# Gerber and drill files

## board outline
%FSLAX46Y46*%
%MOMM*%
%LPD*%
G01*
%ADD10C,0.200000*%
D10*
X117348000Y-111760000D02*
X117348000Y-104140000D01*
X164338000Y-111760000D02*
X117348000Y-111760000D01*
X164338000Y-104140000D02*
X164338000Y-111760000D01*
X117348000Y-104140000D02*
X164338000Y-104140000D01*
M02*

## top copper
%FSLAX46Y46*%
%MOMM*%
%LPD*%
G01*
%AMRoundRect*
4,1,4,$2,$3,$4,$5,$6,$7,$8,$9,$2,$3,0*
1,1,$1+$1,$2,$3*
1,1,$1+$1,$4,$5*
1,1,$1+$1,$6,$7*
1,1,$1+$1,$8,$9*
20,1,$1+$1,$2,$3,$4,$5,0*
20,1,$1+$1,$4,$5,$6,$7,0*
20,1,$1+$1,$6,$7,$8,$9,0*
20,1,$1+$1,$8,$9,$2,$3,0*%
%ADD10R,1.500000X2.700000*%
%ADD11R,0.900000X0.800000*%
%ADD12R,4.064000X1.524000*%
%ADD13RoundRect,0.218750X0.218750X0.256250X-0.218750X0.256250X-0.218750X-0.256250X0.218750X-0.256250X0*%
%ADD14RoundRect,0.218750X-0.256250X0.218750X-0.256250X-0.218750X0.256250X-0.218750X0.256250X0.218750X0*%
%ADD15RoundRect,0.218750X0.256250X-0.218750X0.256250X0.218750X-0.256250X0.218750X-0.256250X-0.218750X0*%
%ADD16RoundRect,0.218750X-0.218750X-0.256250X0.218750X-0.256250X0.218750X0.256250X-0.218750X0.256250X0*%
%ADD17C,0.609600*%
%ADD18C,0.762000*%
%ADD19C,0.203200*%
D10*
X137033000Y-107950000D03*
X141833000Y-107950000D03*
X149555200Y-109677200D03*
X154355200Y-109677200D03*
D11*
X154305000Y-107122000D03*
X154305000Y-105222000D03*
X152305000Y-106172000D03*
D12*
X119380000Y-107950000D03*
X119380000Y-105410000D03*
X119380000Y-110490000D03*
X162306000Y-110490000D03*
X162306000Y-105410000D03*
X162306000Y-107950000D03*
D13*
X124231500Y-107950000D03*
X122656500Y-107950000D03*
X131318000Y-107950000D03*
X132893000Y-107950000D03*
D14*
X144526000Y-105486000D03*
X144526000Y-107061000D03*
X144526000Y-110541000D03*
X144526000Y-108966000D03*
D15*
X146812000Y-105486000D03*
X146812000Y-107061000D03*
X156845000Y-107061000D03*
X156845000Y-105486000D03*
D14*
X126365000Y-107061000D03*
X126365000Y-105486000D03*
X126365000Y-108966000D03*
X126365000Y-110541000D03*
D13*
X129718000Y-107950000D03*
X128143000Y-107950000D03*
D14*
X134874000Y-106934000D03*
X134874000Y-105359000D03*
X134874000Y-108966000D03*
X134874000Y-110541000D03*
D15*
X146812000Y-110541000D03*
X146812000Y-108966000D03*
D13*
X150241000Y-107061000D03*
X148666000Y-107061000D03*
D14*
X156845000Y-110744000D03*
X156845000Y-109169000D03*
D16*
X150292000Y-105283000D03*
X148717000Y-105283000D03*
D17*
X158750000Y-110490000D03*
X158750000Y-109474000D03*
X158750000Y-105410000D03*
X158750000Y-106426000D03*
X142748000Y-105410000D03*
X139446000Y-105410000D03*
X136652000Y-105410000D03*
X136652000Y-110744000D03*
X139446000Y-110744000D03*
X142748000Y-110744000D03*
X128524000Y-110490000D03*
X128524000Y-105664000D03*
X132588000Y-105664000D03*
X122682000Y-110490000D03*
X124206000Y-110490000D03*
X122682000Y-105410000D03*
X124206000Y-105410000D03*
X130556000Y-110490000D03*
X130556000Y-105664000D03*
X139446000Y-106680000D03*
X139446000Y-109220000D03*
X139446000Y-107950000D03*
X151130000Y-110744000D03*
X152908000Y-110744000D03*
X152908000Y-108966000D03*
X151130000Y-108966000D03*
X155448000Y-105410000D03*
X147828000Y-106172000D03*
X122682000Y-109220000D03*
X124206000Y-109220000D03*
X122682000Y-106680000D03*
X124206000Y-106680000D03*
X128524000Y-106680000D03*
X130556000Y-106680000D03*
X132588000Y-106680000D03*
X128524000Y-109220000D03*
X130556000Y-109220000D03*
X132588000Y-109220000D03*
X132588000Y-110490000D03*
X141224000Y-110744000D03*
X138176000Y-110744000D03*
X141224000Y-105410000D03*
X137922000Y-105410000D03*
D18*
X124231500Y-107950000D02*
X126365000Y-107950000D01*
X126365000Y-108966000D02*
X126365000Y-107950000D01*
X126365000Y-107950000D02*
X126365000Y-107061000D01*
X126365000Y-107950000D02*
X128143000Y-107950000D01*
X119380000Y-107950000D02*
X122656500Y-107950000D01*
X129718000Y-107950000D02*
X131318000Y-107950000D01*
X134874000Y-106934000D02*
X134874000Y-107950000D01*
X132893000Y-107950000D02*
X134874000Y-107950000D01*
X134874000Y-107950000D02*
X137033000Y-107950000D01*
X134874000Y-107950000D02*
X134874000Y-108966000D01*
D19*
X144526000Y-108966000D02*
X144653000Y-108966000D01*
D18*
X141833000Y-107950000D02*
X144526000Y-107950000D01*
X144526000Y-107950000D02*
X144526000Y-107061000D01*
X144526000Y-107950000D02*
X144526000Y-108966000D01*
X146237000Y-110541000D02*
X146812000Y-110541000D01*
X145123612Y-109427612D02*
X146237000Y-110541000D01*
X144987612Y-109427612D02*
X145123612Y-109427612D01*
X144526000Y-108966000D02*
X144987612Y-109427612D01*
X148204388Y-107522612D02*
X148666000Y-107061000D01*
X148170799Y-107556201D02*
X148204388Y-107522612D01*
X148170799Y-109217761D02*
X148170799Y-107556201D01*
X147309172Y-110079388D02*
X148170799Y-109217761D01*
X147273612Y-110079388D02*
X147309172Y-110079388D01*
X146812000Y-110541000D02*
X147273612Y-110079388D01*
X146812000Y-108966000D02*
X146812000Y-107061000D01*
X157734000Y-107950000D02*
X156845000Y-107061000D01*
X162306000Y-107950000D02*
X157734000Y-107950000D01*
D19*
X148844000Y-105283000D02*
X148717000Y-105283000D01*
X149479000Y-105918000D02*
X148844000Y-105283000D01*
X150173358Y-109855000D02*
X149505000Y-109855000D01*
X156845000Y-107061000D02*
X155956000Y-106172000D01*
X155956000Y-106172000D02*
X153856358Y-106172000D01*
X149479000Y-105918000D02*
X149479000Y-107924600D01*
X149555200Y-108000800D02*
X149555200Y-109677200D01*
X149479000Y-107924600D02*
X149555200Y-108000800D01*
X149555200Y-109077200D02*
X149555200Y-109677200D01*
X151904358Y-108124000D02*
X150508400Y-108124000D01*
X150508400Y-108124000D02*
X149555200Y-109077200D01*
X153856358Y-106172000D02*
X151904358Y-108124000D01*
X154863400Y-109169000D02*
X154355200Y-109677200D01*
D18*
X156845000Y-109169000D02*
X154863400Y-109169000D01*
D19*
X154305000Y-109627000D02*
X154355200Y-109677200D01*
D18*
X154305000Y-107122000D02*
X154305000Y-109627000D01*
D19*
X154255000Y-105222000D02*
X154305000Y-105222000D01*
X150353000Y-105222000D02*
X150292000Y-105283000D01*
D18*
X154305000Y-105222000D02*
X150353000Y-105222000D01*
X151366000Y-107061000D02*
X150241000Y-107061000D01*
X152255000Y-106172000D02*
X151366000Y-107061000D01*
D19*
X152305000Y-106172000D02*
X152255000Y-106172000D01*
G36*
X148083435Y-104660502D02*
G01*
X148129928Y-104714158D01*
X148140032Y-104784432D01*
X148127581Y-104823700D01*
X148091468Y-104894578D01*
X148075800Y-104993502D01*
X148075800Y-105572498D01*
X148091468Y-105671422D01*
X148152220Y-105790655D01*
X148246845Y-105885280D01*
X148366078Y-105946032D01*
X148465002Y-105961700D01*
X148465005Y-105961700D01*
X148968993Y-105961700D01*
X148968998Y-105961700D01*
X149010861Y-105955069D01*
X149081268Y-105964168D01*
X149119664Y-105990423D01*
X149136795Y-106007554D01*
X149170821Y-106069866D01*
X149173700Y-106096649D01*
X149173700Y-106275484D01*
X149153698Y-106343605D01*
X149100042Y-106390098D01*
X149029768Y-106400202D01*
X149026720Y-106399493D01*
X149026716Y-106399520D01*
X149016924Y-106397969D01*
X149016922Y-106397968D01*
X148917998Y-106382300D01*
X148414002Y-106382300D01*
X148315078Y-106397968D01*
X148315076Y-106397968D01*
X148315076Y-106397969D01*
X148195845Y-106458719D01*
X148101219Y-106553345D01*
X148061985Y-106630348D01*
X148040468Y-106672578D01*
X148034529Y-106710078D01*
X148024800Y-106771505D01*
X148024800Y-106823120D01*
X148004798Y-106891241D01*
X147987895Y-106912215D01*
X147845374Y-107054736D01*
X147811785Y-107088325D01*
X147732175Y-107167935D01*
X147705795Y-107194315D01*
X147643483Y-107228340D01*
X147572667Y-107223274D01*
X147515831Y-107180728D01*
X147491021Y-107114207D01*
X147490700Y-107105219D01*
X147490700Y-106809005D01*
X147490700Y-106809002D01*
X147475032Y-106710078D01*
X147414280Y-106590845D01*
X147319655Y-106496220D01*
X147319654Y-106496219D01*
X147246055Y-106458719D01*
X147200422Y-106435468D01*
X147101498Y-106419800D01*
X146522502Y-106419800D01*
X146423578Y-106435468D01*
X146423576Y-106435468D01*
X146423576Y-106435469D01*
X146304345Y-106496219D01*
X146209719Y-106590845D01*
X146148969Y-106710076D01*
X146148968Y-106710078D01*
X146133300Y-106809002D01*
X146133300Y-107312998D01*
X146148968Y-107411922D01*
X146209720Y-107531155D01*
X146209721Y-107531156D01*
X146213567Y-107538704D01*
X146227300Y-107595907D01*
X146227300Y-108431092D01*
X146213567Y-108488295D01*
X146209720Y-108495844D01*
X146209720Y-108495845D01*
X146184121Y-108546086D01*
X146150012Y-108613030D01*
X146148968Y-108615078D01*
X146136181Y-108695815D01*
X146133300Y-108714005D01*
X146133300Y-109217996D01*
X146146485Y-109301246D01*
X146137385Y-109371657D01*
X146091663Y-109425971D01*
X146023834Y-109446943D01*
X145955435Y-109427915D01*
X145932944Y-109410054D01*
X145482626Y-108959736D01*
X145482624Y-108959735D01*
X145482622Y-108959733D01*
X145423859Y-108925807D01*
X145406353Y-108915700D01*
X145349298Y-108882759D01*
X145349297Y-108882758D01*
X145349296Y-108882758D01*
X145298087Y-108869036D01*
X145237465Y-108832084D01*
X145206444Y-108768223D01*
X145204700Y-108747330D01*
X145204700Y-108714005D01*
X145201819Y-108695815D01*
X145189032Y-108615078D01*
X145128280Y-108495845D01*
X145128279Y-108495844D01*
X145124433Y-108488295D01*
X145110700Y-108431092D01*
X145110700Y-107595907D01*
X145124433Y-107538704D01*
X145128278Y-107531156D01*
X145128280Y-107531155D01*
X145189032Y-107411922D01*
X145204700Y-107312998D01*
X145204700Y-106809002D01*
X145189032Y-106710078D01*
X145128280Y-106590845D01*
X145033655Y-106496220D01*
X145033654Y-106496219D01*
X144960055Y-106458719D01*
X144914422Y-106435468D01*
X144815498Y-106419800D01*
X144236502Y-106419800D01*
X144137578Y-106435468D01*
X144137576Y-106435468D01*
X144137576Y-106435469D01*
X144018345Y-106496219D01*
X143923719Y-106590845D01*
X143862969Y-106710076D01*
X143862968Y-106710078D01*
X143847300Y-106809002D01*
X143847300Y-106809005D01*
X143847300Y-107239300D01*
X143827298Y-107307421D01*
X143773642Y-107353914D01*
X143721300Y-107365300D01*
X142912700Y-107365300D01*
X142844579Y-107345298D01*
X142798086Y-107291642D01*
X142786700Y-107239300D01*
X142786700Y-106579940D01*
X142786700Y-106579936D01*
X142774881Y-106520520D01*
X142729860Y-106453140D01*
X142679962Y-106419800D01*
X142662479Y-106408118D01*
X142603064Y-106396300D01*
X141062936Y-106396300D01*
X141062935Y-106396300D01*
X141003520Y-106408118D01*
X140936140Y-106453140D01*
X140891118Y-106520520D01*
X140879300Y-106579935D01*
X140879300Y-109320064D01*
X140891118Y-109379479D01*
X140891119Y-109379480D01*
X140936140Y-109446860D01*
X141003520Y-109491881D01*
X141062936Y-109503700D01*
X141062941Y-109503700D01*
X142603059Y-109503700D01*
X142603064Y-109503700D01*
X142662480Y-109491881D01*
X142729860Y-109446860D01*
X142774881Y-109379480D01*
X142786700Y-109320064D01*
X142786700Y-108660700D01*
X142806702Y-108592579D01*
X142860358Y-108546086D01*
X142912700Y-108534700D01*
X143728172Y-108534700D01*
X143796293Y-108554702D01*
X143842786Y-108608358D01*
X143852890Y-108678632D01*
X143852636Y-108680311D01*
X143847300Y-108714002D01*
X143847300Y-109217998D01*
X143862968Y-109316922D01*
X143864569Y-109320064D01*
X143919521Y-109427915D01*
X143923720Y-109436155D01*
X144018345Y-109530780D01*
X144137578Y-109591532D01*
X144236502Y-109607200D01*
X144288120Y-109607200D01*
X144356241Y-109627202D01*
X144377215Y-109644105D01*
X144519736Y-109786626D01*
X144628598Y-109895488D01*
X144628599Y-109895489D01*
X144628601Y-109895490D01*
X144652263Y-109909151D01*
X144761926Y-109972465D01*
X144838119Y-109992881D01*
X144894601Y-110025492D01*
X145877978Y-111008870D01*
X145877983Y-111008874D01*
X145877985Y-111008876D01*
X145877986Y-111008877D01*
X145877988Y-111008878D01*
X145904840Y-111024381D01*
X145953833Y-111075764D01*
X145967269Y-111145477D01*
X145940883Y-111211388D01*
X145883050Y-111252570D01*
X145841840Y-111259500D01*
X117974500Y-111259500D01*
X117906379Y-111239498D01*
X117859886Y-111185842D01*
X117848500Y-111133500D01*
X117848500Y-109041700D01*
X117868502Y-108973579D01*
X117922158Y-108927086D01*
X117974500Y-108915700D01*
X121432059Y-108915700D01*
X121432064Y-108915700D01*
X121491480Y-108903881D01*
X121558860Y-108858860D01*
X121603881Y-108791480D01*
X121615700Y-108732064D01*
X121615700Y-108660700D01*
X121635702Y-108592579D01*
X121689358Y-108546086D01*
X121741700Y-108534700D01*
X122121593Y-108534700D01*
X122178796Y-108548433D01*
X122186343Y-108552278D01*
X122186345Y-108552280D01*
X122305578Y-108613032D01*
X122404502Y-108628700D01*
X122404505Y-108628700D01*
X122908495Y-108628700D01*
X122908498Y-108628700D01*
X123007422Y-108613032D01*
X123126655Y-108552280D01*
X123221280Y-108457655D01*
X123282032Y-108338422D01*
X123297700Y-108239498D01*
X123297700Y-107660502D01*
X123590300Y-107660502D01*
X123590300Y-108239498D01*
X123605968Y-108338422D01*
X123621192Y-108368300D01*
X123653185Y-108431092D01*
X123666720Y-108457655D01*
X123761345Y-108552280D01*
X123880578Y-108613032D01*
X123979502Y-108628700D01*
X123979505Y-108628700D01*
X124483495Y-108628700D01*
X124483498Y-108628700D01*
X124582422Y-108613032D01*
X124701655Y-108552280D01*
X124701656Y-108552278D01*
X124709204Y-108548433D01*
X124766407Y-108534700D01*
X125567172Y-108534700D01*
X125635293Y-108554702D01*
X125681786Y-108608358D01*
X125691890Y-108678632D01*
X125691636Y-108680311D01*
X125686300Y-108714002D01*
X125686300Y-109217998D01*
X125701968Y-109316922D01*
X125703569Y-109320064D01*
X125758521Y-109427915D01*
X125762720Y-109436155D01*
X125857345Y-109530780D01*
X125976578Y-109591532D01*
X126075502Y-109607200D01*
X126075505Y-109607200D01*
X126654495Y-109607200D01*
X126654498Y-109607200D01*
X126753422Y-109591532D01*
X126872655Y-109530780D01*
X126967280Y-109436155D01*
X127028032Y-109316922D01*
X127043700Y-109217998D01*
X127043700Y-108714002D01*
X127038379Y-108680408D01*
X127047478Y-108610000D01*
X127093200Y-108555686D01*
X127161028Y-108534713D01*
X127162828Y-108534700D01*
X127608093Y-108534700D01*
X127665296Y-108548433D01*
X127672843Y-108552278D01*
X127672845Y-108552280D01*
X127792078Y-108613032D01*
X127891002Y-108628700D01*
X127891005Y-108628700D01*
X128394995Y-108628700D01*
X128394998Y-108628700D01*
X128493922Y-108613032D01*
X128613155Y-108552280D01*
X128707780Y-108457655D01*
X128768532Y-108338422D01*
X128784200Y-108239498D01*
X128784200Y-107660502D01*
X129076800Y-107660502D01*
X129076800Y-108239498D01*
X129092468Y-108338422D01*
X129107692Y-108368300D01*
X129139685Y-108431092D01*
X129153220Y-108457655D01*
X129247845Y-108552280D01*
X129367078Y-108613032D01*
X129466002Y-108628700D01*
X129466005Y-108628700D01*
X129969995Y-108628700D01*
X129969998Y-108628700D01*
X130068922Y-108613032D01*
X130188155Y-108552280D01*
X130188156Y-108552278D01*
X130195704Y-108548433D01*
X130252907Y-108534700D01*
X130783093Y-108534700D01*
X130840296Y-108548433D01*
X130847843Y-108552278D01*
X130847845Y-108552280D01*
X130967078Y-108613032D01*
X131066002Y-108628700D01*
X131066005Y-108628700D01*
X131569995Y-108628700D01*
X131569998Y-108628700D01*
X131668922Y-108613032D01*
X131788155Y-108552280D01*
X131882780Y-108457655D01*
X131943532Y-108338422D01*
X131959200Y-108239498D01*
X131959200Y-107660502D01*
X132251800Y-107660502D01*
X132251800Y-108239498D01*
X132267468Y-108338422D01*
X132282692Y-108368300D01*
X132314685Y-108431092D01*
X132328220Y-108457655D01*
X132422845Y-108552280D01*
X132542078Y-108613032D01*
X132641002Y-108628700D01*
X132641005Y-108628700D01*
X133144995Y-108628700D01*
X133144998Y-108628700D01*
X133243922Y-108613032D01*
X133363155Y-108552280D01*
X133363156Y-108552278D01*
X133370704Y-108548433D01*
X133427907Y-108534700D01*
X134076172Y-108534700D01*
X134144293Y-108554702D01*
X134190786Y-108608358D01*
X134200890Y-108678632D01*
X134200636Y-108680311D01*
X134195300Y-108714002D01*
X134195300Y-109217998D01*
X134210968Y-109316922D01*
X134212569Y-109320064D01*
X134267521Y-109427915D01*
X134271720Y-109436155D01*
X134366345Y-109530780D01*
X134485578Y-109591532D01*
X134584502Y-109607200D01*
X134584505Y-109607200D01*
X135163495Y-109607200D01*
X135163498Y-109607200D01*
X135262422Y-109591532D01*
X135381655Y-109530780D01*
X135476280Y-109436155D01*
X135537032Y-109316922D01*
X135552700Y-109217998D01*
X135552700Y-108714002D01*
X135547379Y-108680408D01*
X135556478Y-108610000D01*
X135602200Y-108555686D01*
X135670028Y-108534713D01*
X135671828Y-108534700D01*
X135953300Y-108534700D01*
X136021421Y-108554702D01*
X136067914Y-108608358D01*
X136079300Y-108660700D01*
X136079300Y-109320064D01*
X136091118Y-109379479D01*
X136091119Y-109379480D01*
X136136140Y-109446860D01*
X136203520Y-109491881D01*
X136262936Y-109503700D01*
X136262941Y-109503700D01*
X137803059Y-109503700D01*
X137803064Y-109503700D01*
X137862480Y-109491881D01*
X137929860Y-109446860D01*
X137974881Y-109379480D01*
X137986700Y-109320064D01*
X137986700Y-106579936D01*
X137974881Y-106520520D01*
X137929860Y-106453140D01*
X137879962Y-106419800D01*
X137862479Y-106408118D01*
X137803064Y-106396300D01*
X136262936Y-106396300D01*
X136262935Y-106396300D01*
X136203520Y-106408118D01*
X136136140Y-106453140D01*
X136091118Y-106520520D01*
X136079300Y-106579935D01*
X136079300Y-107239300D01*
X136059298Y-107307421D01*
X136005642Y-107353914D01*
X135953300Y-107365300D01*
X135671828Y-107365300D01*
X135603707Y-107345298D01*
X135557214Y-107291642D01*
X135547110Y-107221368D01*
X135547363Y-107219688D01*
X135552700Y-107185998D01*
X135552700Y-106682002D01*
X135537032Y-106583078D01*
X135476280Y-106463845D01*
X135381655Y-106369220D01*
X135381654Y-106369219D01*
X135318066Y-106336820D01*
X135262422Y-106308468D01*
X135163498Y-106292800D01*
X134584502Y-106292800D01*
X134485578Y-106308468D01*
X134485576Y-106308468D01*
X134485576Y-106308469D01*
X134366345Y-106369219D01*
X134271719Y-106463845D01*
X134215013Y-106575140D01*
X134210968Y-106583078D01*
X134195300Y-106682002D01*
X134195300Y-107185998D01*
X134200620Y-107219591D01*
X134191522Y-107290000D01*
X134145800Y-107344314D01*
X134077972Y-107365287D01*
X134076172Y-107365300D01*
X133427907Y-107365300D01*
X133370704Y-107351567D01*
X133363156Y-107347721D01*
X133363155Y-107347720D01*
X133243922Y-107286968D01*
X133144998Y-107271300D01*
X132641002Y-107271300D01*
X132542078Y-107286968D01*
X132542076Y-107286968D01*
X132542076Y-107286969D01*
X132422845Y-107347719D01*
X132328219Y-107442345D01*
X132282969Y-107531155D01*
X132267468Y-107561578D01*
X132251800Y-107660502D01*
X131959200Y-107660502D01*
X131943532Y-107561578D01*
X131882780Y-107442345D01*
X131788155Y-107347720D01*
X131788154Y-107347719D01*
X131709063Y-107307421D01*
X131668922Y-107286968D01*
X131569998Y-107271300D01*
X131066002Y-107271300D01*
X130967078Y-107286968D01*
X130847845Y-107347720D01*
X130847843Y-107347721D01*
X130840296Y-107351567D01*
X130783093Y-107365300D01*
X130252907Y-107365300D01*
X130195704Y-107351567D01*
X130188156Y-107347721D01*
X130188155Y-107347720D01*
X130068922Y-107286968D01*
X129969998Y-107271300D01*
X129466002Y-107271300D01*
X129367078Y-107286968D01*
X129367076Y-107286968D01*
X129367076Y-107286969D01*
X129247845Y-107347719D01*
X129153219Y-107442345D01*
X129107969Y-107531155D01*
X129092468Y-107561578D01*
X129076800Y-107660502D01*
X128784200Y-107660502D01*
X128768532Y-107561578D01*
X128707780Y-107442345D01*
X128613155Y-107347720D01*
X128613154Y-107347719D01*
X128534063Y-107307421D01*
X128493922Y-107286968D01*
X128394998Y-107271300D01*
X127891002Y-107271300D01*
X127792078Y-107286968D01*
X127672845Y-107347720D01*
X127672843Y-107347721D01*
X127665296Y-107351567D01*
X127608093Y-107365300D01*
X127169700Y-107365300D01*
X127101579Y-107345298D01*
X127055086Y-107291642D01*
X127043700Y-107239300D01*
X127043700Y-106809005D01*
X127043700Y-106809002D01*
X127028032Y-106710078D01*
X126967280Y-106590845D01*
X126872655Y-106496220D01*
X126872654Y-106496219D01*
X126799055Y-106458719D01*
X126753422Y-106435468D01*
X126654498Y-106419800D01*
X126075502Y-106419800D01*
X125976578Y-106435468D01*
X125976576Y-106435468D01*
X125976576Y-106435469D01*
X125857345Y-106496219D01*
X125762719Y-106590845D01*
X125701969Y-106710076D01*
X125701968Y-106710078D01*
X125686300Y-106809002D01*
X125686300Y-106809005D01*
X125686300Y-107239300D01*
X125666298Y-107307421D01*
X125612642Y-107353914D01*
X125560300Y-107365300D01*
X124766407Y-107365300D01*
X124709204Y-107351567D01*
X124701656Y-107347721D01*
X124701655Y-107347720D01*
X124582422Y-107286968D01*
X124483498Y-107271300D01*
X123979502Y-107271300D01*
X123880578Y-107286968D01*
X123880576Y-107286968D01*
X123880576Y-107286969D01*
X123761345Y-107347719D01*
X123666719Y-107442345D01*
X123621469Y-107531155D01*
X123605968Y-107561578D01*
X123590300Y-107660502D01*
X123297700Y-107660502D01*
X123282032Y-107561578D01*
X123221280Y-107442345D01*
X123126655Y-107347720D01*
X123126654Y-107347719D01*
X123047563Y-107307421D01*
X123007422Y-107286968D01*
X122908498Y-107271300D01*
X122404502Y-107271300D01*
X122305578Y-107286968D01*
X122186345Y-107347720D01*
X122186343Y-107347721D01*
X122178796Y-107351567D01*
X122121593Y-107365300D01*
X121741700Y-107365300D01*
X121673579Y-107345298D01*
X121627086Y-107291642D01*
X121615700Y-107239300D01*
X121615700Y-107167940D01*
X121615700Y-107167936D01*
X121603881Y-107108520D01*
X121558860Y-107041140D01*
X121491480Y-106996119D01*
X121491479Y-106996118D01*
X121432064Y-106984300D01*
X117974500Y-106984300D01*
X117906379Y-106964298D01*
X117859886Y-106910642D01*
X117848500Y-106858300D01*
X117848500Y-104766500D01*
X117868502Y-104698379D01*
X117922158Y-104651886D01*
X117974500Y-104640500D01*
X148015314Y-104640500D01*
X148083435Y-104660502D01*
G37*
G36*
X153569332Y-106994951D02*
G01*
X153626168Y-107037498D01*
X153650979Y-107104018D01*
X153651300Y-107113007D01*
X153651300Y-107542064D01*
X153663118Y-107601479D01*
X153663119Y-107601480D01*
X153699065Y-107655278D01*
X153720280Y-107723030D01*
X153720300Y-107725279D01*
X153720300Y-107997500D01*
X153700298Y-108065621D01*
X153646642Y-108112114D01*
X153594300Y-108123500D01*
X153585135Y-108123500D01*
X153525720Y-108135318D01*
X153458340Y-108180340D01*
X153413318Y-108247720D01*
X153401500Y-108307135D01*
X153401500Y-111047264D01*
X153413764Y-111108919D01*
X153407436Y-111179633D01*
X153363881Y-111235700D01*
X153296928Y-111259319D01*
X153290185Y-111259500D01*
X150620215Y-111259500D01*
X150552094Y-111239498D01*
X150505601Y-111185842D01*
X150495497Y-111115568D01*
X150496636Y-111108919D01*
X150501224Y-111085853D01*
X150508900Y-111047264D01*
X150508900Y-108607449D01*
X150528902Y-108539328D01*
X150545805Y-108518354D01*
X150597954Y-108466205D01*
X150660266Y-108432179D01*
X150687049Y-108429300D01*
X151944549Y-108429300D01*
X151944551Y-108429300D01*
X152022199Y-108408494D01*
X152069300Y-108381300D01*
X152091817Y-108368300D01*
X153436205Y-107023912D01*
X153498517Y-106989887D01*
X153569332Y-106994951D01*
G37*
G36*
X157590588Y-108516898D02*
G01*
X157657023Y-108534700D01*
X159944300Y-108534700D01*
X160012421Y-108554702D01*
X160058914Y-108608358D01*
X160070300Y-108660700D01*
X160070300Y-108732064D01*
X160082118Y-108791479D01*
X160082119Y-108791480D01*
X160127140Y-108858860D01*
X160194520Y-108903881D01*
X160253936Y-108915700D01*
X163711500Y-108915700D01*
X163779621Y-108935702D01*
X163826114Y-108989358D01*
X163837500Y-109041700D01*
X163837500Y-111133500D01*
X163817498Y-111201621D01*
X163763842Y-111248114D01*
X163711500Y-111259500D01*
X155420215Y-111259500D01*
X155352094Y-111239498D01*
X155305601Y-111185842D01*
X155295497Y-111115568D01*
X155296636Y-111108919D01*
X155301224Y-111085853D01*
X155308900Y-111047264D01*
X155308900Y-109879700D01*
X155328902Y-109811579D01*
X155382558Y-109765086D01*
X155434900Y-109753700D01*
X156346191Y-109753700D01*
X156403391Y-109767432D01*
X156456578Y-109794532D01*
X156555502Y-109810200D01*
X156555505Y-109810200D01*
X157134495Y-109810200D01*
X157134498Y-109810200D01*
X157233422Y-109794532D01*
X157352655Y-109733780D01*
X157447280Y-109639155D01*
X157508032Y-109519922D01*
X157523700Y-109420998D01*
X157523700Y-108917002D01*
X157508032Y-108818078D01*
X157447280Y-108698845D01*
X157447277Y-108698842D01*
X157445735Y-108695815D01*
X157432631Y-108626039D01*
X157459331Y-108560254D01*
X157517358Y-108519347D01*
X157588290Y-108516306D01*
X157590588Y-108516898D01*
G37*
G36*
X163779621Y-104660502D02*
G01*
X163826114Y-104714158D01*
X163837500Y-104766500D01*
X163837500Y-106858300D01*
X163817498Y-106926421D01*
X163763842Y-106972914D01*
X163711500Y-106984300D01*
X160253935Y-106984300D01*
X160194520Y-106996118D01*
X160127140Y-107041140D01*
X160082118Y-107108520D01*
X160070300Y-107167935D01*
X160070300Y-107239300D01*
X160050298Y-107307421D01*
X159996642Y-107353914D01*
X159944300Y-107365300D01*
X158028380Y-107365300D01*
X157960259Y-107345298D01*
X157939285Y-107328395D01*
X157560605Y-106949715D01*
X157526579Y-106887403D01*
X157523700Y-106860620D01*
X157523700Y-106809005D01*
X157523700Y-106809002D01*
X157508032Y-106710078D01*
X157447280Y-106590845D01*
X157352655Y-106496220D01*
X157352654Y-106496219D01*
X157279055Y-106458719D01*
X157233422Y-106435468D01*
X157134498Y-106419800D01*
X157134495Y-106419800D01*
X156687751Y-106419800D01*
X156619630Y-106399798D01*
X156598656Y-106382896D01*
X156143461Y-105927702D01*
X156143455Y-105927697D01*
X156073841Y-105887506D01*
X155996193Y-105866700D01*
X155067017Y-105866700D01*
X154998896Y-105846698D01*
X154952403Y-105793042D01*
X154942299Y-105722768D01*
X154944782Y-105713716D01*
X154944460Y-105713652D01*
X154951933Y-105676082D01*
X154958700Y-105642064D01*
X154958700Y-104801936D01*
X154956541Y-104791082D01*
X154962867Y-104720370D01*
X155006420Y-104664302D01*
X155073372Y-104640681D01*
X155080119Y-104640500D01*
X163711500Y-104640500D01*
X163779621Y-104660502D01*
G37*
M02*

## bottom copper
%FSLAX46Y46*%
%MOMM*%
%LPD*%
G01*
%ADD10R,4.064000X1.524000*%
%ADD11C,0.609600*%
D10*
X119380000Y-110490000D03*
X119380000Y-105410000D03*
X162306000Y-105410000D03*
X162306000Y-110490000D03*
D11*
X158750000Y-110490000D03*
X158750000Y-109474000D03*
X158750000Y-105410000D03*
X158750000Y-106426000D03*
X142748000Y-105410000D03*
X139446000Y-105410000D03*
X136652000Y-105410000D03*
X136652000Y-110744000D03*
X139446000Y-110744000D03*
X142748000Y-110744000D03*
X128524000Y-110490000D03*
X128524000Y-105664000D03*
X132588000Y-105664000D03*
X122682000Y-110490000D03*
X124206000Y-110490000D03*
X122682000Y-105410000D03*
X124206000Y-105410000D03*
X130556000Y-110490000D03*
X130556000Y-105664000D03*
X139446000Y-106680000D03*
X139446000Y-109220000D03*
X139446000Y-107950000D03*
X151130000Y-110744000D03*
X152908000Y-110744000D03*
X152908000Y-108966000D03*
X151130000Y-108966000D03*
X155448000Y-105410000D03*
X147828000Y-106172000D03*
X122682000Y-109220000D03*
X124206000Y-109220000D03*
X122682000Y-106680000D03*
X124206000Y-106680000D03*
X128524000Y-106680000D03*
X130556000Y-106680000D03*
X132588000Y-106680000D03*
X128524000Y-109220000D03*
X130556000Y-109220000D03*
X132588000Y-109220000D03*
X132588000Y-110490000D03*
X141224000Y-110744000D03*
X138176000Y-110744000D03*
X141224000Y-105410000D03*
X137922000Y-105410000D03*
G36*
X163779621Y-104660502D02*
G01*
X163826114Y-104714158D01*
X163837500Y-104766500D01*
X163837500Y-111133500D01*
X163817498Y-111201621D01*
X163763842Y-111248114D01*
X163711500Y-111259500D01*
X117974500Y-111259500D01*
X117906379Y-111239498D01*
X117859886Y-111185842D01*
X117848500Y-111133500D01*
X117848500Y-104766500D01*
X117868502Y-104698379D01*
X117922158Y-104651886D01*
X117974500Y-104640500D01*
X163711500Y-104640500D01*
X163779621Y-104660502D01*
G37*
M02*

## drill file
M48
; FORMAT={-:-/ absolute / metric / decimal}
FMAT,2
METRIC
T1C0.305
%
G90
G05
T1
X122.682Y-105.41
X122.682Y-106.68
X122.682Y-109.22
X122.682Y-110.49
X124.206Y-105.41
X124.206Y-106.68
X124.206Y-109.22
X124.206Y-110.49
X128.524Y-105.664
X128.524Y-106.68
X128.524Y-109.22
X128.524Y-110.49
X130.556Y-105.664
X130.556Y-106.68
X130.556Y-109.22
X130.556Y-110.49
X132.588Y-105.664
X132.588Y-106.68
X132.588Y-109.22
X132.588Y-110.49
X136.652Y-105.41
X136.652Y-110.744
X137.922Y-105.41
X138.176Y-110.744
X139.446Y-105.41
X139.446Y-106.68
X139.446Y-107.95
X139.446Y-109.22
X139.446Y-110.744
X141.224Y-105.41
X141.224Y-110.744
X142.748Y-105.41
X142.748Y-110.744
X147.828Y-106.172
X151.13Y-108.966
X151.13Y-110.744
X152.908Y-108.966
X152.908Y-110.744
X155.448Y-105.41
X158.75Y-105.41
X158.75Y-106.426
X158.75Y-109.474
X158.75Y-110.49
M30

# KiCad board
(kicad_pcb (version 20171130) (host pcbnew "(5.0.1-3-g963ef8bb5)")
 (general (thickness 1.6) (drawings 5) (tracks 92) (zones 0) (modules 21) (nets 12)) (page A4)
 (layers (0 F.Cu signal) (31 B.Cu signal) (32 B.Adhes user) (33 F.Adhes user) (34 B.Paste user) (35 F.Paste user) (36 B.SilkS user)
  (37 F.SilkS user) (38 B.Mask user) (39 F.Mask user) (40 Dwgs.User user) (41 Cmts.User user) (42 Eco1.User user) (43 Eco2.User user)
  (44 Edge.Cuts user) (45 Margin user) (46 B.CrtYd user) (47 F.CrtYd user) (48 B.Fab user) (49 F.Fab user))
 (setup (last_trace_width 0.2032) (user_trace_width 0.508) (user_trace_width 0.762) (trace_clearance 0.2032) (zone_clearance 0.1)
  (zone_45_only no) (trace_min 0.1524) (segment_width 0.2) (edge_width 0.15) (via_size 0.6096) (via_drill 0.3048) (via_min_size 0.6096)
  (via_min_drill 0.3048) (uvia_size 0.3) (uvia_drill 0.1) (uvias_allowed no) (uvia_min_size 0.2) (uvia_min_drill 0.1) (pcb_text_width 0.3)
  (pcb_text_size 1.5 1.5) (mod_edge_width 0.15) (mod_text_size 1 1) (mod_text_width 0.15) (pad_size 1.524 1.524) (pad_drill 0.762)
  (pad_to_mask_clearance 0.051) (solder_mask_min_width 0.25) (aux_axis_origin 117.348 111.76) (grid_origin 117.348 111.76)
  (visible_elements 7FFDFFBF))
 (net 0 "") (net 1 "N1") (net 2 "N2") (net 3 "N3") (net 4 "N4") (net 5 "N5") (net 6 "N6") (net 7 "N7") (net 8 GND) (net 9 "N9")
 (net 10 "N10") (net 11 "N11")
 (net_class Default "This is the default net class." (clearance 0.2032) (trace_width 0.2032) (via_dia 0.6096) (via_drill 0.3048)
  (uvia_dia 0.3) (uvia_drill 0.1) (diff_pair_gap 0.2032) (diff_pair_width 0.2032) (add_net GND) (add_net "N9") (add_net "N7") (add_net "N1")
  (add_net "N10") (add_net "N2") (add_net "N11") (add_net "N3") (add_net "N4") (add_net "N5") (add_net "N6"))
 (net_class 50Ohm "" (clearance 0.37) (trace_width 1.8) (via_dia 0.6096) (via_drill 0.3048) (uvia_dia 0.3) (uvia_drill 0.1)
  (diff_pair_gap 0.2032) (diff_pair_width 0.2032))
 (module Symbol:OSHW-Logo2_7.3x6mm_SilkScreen (layer B.Cu) (at 155.194 107.696 180)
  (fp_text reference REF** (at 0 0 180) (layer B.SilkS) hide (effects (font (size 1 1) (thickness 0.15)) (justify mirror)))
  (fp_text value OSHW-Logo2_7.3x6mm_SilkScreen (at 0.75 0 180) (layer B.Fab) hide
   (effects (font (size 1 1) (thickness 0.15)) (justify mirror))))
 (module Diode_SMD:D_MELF (layer F.Cu) (at 139.433 107.95 180)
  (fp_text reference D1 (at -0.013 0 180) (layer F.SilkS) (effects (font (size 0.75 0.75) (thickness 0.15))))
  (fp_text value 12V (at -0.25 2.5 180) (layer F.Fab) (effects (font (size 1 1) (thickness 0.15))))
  (pad 2 smd rect (at 2.4 0 180) (size 1.5 2.7) (layers F.Cu F.Paste F.Mask) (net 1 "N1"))
  (pad 1 smd rect (at -2.4 0 180) (size 1.5 2.7) (layers F.Cu F.Paste F.Mask) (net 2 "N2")))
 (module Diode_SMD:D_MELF (layer F.Cu) (at 151.9552 109.6772)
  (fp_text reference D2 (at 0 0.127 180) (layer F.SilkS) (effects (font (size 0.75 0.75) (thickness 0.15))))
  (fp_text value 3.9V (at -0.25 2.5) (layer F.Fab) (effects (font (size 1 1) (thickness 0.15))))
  (pad 1 smd rect (at -2.4 0) (size 1.5 2.7) (layers F.Cu F.Paste F.Mask) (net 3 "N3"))
  (pad 2 smd rect (at 2.4 0) (size 1.5 2.7) (layers F.Cu F.Paste F.Mask) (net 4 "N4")))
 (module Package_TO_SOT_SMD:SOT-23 (layer F.Cu) (at 153.305 106.172 180)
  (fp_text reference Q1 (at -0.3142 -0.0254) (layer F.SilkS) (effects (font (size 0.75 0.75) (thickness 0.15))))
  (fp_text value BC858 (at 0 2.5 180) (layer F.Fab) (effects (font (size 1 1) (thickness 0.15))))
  (pad 1 smd rect (at -1 -0.95 180) (size 0.9 0.8) (layers F.Cu F.Paste F.Mask) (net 4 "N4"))
  (pad 2 smd rect (at -1 0.95 180) (size 0.9 0.8) (layers F.Cu F.Paste F.Mask) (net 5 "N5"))
  (pad 3 smd rect (at 1 0 180) (size 0.9 0.8) (layers F.Cu F.Paste F.Mask) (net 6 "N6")))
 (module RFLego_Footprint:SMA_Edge (layer F.Cu) (at 117.348 107.95)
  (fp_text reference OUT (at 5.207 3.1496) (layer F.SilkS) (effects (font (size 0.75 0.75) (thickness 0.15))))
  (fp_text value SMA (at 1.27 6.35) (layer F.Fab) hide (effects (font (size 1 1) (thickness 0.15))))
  (pad 1 smd rect (at 2.032 0) (size 4.064 1.524) (layers F.Cu F.Mask) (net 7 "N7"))
  (pad 2 smd rect (at 2.032 -2.54) (size 4.064 1.524) (layers F.Cu F.Mask) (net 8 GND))
  (pad 2 smd rect (at 2.032 2.54) (size 4.064 1.524) (layers B.Cu B.Mask) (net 8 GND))
  (pad 2 smd rect (at 2.032 -2.54) (size 4.064 1.524) (layers B.Cu B.Mask) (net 8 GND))
  (pad 2 smd rect (at 2.032 2.54) (size 4.064 1.524) (layers F.Cu F.Mask) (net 8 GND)))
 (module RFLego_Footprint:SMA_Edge (layer F.Cu) (at 160.274 107.95)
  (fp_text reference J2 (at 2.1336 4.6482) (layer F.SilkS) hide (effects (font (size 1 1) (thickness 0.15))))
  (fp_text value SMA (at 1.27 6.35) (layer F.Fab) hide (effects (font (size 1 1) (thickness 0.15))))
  (pad 2 smd rect (at 2.032 2.54) (size 4.064 1.524) (layers F.Cu F.Mask) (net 8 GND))
  (pad 2 smd rect (at 2.032 -2.54) (size 4.064 1.524) (layers B.Cu B.Mask) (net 8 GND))
  (pad 2 smd rect (at 2.032 2.54) (size 4.064 1.524) (layers B.Cu B.Mask) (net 8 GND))
  (pad 2 smd rect (at 2.032 -2.54) (size 4.064 1.524) (layers F.Cu F.Mask) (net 8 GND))
  (pad 1 smd rect (at 2.032 0) (size 4.064 1.524) (layers F.Cu F.Mask) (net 3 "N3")))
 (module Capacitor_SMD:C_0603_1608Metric (layer F.Cu) (at 123.444 107.95 180)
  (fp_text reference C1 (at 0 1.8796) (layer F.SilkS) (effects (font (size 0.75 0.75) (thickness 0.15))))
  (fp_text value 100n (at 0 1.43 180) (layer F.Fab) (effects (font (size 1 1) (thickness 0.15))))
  (pad 1 smd roundrect (at -0.7875 0 180) (size 0.875 0.95) (layers F.Cu F.Paste F.Mask) (roundrect_rratio 0.25) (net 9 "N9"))
  (pad 2 smd roundrect (at 0.7875 0 180) (size 0.875 0.95) (layers F.Cu F.Paste F.Mask) (roundrect_rratio 0.25) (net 7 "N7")))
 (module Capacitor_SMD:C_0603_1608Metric (layer F.Cu) (at 132.1055 107.95 180)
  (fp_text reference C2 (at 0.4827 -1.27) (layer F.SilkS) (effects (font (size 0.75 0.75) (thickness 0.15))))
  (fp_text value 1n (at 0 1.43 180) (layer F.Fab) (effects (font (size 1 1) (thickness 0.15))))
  (pad 2 smd roundrect (at 0.7875 0 180) (size 0.875 0.95) (layers F.Cu F.Paste F.Mask) (roundrect_rratio 0.25) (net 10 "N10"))
  (pad 1 smd roundrect (at -0.7875 0 180) (size 0.875 0.95) (layers F.Cu F.Paste F.Mask) (roundrect_rratio 0.25) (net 1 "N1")))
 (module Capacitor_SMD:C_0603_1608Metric (layer F.Cu) (at 144.526 106.2735 270)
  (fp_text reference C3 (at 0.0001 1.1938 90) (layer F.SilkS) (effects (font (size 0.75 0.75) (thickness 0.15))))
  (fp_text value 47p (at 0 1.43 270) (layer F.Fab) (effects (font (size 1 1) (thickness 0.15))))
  (pad 1 smd roundrect (at -0.7875 0 270) (size 0.875 0.95) (layers F.Cu F.Paste F.Mask) (roundrect_rratio 0.25) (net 8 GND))
  (pad 2 smd roundrect (at 0.7875 0 270) (size 0.875 0.95) (layers F.Cu F.Paste F.Mask) (roundrect_rratio 0.25) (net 2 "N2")))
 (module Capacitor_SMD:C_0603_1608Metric (layer F.Cu) (at 144.526 109.7535 270)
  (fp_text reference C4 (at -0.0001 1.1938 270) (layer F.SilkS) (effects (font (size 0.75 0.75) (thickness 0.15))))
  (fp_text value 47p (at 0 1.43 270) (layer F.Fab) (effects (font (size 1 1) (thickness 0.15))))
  (pad 2 smd roundrect (at 0.7875 0 270) (size 0.875 0.95) (layers F.Cu F.Paste F.Mask) (roundrect_rratio 0.25) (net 8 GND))
  (pad 1 smd roundrect (at -0.7875 0 270) (size 0.875 0.95) (layers F.Cu F.Paste F.Mask) (roundrect_rratio 0.25) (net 2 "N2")))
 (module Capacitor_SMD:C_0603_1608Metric (layer F.Cu) (at 146.812 106.2735 90)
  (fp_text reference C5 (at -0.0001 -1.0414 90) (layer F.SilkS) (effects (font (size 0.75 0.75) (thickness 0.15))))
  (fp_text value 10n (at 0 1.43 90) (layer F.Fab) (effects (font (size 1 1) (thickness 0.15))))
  (pad 2 smd roundrect (at 0.7875 0 90) (size 0.875 0.95) (layers F.Cu F.Paste F.Mask) (roundrect_rratio 0.25) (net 8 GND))
  (pad 1 smd roundrect (at -0.7875 0 90) (size 0.875 0.95) (layers F.Cu F.Paste F.Mask) (roundrect_rratio 0.25) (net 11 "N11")))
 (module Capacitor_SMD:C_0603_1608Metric (layer F.Cu) (at 156.845 106.2735 90)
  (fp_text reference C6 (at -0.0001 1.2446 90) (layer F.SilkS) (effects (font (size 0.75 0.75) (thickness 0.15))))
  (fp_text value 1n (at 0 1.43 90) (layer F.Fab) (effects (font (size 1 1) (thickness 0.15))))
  (pad 1 smd roundrect (at -0.7875 0 90) (size 0.875 0.95) (layers F.Cu F.Paste F.Mask) (roundrect_rratio 0.25) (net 3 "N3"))
  (pad 2 smd roundrect (at 0.7875 0 90) (size 0.875 0.95) (layers F.Cu F.Paste F.Mask) (roundrect_rratio 0.25) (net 8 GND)))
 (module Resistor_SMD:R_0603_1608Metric (layer F.Cu) (at 126.365 106.2735 270)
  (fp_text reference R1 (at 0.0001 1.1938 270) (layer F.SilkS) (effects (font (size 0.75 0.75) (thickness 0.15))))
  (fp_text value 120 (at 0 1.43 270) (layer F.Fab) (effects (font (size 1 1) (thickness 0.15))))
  (pad 2 smd roundrect (at 0.7875 0 270) (size 0.875 0.95) (layers F.Cu F.Paste F.Mask) (roundrect_rratio 0.25) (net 9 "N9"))
  (pad 1 smd roundrect (at -0.7875 0 270) (size 0.875 0.95) (layers F.Cu F.Paste F.Mask) (roundrect_rratio 0.25) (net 8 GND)))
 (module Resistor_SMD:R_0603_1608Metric (layer F.Cu) (at 126.365 109.7535 270)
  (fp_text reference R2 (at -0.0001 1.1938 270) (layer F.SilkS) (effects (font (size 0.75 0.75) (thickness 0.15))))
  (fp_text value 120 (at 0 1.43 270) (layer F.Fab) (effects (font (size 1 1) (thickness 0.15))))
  (pad 1 smd roundrect (at -0.7875 0 270) (size 0.875 0.95) (layers F.Cu F.Paste F.Mask) (roundrect_rratio 0.25) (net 9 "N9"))
  (pad 2 smd roundrect (at 0.7875 0 270) (size 0.875 0.95) (layers F.Cu F.Paste F.Mask) (roundrect_rratio 0.25) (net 8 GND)))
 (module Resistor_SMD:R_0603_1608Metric (layer F.Cu) (at 128.9305 107.95 180)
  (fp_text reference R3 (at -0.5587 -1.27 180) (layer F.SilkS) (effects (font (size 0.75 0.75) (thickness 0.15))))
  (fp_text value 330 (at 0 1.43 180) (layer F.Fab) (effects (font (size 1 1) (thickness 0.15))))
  (pad 1 smd roundrect (at -0.7875 0 180) (size 0.875 0.95) (layers F.Cu F.Paste F.Mask) (roundrect_rratio 0.25) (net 10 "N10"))
  (pad 2 smd roundrect (at 0.7875 0 180) (size 0.875 0.95) (layers F.Cu F.Paste F.Mask) (roundrect_rratio 0.25) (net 9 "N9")))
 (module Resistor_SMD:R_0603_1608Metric (layer F.Cu) (at 134.874 106.1465 270)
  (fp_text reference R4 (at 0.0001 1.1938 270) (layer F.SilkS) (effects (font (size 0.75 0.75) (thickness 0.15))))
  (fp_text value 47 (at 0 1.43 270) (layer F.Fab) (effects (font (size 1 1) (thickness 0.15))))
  (pad 2 smd roundrect (at 0.7875 0 270) (size 0.875 0.95) (layers F.Cu F.Paste F.Mask) (roundrect_rratio 0.25) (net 1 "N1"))
  (pad 1 smd roundrect (at -0.7875 0 270) (size 0.875 0.95) (layers F.Cu F.Paste F.Mask) (roundrect_rratio 0.25) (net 8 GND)))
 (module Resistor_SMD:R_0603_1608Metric (layer F.Cu) (at 134.874 109.7535 270)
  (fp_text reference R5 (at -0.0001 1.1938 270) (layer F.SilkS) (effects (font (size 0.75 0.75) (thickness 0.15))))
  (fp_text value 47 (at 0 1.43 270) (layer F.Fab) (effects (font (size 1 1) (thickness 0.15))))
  (pad 1 smd roundrect (at -0.7875 0 270) (size 0.875 0.95) (layers F.Cu F.Paste F.Mask) (roundrect_rratio 0.25) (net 1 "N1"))
  (pad 2 smd roundrect (at 0.7875 0 270) (size 0.875 0.95) (layers F.Cu F.Paste F.Mask) (roundrect_rratio 0.25) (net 8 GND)))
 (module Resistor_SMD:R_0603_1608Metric (layer F.Cu) (at 146.812 109.7535 90)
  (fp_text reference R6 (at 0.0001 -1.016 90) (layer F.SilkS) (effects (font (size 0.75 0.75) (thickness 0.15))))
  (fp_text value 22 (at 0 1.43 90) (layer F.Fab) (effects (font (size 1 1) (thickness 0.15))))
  (pad 1 smd roundrect (at -0.7875 0 90) (size 0.875 0.95) (layers F.Cu F.Paste F.Mask) (roundrect_rratio 0.25) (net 2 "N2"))
  (pad 2 smd roundrect (at 0.7875 0 90) (size 0.875 0.95) (layers F.Cu F.Paste F.Mask) (roundrect_rratio 0.25) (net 11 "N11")))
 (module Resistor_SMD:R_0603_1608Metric (layer F.Cu) (at 149.4535 107.061 180)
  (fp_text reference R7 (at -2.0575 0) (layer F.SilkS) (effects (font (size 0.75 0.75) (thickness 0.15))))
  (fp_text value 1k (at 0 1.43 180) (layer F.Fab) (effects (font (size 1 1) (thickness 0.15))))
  (pad 1 smd roundrect (at -0.7875 0 180) (size 0.875 0.95) (layers F.Cu F.Paste F.Mask) (roundrect_rratio 0.25) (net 6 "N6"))
  (pad 2 smd roundrect (at 0.7875 0 180) (size 0.875 0.95) (layers F.Cu F.Paste F.Mask) (roundrect_rratio 0.25) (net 2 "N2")))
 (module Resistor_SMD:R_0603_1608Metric (layer F.Cu) (at 156.845 109.9565 270)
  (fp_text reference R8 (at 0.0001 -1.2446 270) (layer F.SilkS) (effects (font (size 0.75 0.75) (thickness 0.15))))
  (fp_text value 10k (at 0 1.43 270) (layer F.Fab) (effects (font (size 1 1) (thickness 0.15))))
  (pad 2 smd roundrect (at 0.7875 0 270) (size 0.875 0.95) (layers F.Cu F.Paste F.Mask) (roundrect_rratio 0.25) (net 8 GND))
  (pad 1 smd roundrect (at -0.7875 0 270) (size 0.875 0.95) (layers F.Cu F.Paste F.Mask) (roundrect_rratio 0.25) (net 4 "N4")))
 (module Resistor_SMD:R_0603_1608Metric (layer F.Cu) (at 149.5045 105.283)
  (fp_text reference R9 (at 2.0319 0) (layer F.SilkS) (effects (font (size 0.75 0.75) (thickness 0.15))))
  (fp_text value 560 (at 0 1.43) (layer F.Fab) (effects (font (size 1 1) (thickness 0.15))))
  (pad 2 smd roundrect (at 0.7875 0) (size 0.875 0.95) (layers F.Cu F.Paste F.Mask) (roundrect_rratio 0.25) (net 5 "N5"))
  (pad 1 smd roundrect (at -0.7875 0) (size 0.875 0.95) (layers F.Cu F.Paste F.Mask) (roundrect_rratio 0.25) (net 3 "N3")))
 (gr_line (start 117.348 111.76) (end 117.348 104.14) (layer Edge.Cuts) (width 0.2))
 (gr_line (start 164.338 111.76) (end 117.348 111.76) (layer Edge.Cuts) (width 0.2))
 (gr_line (start 164.338 104.14) (end 164.338 111.76) (layer Edge.Cuts) (width 0.2))
 (gr_line (start 117.348 104.14) (end 164.338 104.14) (layer Edge.Cuts) (width 0.2))
 (segment (start 124.2315 107.95) (end 126.365 107.95) (width 0.762) (layer F.Cu) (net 9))
 (segment (start 126.365 108.966) (end 126.365 107.95) (width 0.762) (layer F.Cu) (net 9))
 (segment (start 126.365 107.95) (end 126.365 107.061) (width 0.762) (layer F.Cu) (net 9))
 (segment (start 126.365 107.95) (end 128.143 107.95) (width 0.762) (layer F.Cu) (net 9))
 (segment (start 119.38 107.95) (end 122.6565 107.95) (width 0.762) (layer F.Cu) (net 7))
 (segment (start 129.718 107.95) (end 131.318 107.95) (width 0.762) (layer F.Cu) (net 10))
 (segment (start 134.874 106.934) (end 134.874 107.95) (width 0.762) (layer F.Cu) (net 1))
 (segment (start 132.893 107.95) (end 134.874 107.95) (width 0.762) (layer F.Cu) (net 1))
 (segment (start 134.874 107.95) (end 137.033 107.95) (width 0.762) (layer F.Cu) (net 1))
 (segment (start 134.874 107.95) (end 134.874 108.966) (width 0.762) (layer F.Cu) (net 1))
 (via (at 158.75 110.49) (size 0.6096) (drill 0.3048) (layers F.Cu B.Cu) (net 8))
 (via (at 158.75 109.474) (size 0.6096) (drill 0.3048) (layers F.Cu B.Cu) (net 8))
 (via (at 158.75 105.41) (size 0.6096) (drill 0.3048) (layers F.Cu B.Cu) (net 8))
 (via (at 158.75 106.426) (size 0.6096) (drill 0.3048) (layers F.Cu B.Cu) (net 8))
 (via (at 142.748 105.41) (size 0.6096) (drill 0.3048) (layers F.Cu B.Cu) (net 8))
 (via (at 139.446 105.41) (size 0.6096) (drill 0.3048) (layers F.Cu B.Cu) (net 8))
 (via (at 136.652 105.41) (size 0.6096) (drill 0.3048) (layers F.Cu B.Cu) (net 8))
 (via (at 136.652 110.744) (size 0.6096) (drill 0.3048) (layers F.Cu B.Cu) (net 8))
 (via (at 139.446 110.744) (size 0.6096) (drill 0.3048) (layers F.Cu B.Cu) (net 8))
 (via (at 142.748 110.744) (size 0.6096) (drill 0.3048) (layers F.Cu B.Cu) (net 8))
 (via (at 128.524 110.49) (size 0.6096) (drill 0.3048) (layers F.Cu B.Cu) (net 8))
 (via (at 128.524 105.664) (size 0.6096) (drill 0.3048) (layers F.Cu B.Cu) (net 8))
 (via (at 132.588 105.664) (size 0.6096) (drill 0.3048) (layers F.Cu B.Cu) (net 8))
 (via (at 122.682 110.49) (size 0.6096) (drill 0.3048) (layers F.Cu B.Cu) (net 8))
 (via (at 124.206 110.49) (size 0.6096) (drill 0.3048) (layers F.Cu B.Cu) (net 8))
 (via (at 122.682 105.41) (size 0.6096) (drill 0.3048) (layers F.Cu B.Cu) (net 8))
 (via (at 124.206 105.41) (size 0.6096) (drill 0.3048) (layers F.Cu B.Cu) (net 8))
 (via (at 130.556 110.49) (size 0.6096) (drill 0.3048) (layers F.Cu B.Cu) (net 8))
 (via (at 130.556 105.664) (size 0.6096) (drill 0.3048) (layers F.Cu B.Cu) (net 8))
 (via (at 139.446 106.68) (size 0.6096) (drill 0.3048) (layers F.Cu B.Cu) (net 8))
 (via (at 139.446 109.22) (size 0.6096) (drill 0.3048) (layers F.Cu B.Cu) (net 8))
 (via (at 139.446 107.95) (size 0.6096) (drill 0.3048) (layers F.Cu B.Cu) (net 8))
 (via (at 151.13 110.744) (size 0.6096) (drill 0.3048) (layers F.Cu B.Cu) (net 8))
 (via (at 152.908 110.744) (size 0.6096) (drill 0.3048) (layers F.Cu B.Cu) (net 8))
 (via (at 152.908 108.966) (size 0.6096) (drill 0.3048) (layers F.Cu B.Cu) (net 8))
 (via (at 151.13 108.966) (size 0.6096) (drill 0.3048) (layers F.Cu B.Cu) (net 8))
 (via (at 155.448 105.41) (size 0.6096) (drill 0.3048) (layers F.Cu B.Cu) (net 8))
 (via (at 147.828 106.172) (size 0.6096) (drill 0.3048) (layers F.Cu B.Cu) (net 8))
 (via (at 122.682 109.22) (size 0.6096) (drill 0.3048) (layers F.Cu B.Cu) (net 8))
 (via (at 124.206 109.22) (size 0.6096) (drill 0.3048) (layers F.Cu B.Cu) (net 8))
 (via (at 122.682 106.68) (size 0.6096) (drill 0.3048) (layers F.Cu B.Cu) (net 8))
 (via (at 124.206 106.68) (size 0.6096) (drill 0.3048) (layers F.Cu B.Cu) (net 8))
 (via (at 128.524 106.68) (size 0.6096) (drill 0.3048) (layers F.Cu B.Cu) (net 8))
 (via (at 130.556 106.68) (size 0.6096) (drill 0.3048) (layers F.Cu B.Cu) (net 8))
 (via (at 132.588 106.68) (size 0.6096) (drill 0.3048) (layers F.Cu B.Cu) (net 8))
 (via (at 128.524 109.22) (size 0.6096) (drill 0.3048) (layers F.Cu B.Cu) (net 8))
 (via (at 130.556 109.22) (size 0.6096) (drill 0.3048) (layers F.Cu B.Cu) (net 8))
 (via (at 132.588 109.22) (size 0.6096) (drill 0.3048) (layers F.Cu B.Cu) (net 8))
 (via (at 132.588 110.49) (size 0.6096) (drill 0.3048) (layers F.Cu B.Cu) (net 8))
 (via (at 141.224 110.744) (size 0.6096) (drill 0.3048) (layers F.Cu B.Cu) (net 8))
 (via (at 138.176 110.744) (size 0.6096) (drill 0.3048) (layers F.Cu B.Cu) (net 8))
 (via (at 141.224 105.41) (size 0.6096) (drill 0.3048) (layers F.Cu B.Cu) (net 8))
 (via (at 137.922 105.41) (size 0.6096) (drill 0.3048) (layers F.Cu B.Cu) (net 8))
 (segment (start 144.526 108.966) (end 144.653 108.966) (width 0.2032) (layer F.Cu) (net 2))
 (segment (start 141.833 107.95) (end 144.526 107.95) (width 0.762) (layer F.Cu) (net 2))
 (segment (start 144.526 107.95) (end 144.526 107.061) (width 0.762) (layer F.Cu) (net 2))
 (segment (start 144.526 107.95) (end 144.526 108.966) (width 0.762) (layer F.Cu) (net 2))
 (segment (start 146.237 110.541) (end 146.812 110.541) (width 0.762) (layer F.Cu) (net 2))
 (segment (start 145.123612 109.427612) (end 146.237 110.541) (width 0.762) (layer F.Cu) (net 2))
 (segment (start 144.987612 109.427612) (end 145.123612 109.427612) (width 0.762) (layer F.Cu) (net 2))
 (segment (start 144.526 108.966) (end 144.987612 109.427612) (width 0.762) (layer F.Cu) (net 2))
 (segment (start 148.204388 107.522612) (end 148.666 107.061) (width 0.762) (layer F.Cu) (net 2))
 (segment (start 148.170799 107.556201) (end 148.204388 107.522612) (width 0.762) (layer F.Cu) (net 2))
 (segment (start 148.170799 109.217761) (end 148.170799 107.556201) (width 0.762) (layer F.Cu) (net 2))
 (segment (start 147.309172 110.079388) (end 148.170799 109.217761) (width 0.762) (layer F.Cu) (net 2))
 (segment (start 147.273612 110.079388) (end 147.309172 110.079388) (width 0.762) (layer F.Cu) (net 2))
 (segment (start 146.812 110.541) (end 147.273612 110.079388) (width 0.762) (layer F.Cu) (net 2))
 (segment (start 146.812 108.966) (end 146.812 107.061) (width 0.762) (layer F.Cu) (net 11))
 (segment (start 157.734 107.95) (end 156.845 107.061) (width 0.762) (layer F.Cu) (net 3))
 (segment (start 162.306 107.95) (end 157.734 107.95) (width 0.762) (layer F.Cu) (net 3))
 (segment (start 148.844 105.283) (end 148.717 105.283) (width 0.2032) (layer F.Cu) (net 3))
 (segment (start 149.479 105.918) (end 148.844 105.283) (width 0.2032) (layer F.Cu) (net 3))
 (segment (start 150.173358 109.855) (end 149.505 109.855) (width 0.2032) (layer F.Cu) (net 3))
 (segment (start 156.845 107.061) (end 155.956 106.172) (width 0.2032) (layer F.Cu) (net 3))
 (segment (start 155.956 106.172) (end 153.856358 106.172) (width 0.2032) (layer F.Cu) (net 3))
 (segment (start 149.479 105.918) (end 149.479 107.9246) (width 0.2032) (layer F.Cu) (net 3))
 (segment (start 149.5552 108.0008) (end 149.5552 109.6772) (width 0.2032) (layer F.Cu) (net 3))
 (segment (start 149.479 107.9246) (end 149.5552 108.0008) (width 0.2032) (layer F.Cu) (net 3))
 (segment (start 149.5552 109.0772) (end 149.5552 109.6772) (width 0.2032) (layer F.Cu) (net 3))
 (segment (start 151.904358 108.124) (end 150.5084 108.124) (width 0.2032) (layer F.Cu) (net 3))
 (segment (start 150.5084 108.124) (end 149.5552 109.0772) (width 0.2032) (layer F.Cu) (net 3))
 (segment (start 153.856358 106.172) (end 151.904358 108.124) (width 0.2032) (layer F.Cu) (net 3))
 (segment (start 154.8634 109.169) (end 154.3552 109.6772) (width 0.2032) (layer F.Cu) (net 4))
 (segment (start 156.845 109.169) (end 154.8634 109.169) (width 0.762) (layer F.Cu) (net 4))
 (segment (start 154.305 109.627) (end 154.3552 109.6772) (width 0.2032) (layer F.Cu) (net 4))
 (segment (start 154.305 107.122) (end 154.305 109.627) (width 0.762) (layer F.Cu) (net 4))
 (segment (start 154.255 105.222) (end 154.305 105.222) (width 0.2032) (layer F.Cu) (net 5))
 (segment (start 150.353 105.222) (end 150.292 105.283) (width 0.2032) (layer F.Cu) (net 5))
 (segment (start 154.305 105.222) (end 150.353 105.222) (width 0.762) (layer F.Cu) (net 5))
 (segment (start 151.366 107.061) (end 150.241 107.061) (width 0.762) (layer F.Cu) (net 6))
 (segment (start 152.255 106.172) (end 151.366 107.061) (width 0.762) (layer F.Cu) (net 6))
 (segment (start 152.305 106.172) (end 152.255 106.172) (width 0.2032) (layer F.Cu) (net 6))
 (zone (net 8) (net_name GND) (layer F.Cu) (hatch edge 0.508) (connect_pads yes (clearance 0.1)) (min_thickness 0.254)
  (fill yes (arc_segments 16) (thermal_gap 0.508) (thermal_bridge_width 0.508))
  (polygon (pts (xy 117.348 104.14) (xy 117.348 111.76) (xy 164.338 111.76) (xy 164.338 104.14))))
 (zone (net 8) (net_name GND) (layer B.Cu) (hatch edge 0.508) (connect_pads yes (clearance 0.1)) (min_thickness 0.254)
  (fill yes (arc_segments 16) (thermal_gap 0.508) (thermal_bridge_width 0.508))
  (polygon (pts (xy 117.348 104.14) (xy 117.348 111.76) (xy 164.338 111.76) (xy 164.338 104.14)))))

